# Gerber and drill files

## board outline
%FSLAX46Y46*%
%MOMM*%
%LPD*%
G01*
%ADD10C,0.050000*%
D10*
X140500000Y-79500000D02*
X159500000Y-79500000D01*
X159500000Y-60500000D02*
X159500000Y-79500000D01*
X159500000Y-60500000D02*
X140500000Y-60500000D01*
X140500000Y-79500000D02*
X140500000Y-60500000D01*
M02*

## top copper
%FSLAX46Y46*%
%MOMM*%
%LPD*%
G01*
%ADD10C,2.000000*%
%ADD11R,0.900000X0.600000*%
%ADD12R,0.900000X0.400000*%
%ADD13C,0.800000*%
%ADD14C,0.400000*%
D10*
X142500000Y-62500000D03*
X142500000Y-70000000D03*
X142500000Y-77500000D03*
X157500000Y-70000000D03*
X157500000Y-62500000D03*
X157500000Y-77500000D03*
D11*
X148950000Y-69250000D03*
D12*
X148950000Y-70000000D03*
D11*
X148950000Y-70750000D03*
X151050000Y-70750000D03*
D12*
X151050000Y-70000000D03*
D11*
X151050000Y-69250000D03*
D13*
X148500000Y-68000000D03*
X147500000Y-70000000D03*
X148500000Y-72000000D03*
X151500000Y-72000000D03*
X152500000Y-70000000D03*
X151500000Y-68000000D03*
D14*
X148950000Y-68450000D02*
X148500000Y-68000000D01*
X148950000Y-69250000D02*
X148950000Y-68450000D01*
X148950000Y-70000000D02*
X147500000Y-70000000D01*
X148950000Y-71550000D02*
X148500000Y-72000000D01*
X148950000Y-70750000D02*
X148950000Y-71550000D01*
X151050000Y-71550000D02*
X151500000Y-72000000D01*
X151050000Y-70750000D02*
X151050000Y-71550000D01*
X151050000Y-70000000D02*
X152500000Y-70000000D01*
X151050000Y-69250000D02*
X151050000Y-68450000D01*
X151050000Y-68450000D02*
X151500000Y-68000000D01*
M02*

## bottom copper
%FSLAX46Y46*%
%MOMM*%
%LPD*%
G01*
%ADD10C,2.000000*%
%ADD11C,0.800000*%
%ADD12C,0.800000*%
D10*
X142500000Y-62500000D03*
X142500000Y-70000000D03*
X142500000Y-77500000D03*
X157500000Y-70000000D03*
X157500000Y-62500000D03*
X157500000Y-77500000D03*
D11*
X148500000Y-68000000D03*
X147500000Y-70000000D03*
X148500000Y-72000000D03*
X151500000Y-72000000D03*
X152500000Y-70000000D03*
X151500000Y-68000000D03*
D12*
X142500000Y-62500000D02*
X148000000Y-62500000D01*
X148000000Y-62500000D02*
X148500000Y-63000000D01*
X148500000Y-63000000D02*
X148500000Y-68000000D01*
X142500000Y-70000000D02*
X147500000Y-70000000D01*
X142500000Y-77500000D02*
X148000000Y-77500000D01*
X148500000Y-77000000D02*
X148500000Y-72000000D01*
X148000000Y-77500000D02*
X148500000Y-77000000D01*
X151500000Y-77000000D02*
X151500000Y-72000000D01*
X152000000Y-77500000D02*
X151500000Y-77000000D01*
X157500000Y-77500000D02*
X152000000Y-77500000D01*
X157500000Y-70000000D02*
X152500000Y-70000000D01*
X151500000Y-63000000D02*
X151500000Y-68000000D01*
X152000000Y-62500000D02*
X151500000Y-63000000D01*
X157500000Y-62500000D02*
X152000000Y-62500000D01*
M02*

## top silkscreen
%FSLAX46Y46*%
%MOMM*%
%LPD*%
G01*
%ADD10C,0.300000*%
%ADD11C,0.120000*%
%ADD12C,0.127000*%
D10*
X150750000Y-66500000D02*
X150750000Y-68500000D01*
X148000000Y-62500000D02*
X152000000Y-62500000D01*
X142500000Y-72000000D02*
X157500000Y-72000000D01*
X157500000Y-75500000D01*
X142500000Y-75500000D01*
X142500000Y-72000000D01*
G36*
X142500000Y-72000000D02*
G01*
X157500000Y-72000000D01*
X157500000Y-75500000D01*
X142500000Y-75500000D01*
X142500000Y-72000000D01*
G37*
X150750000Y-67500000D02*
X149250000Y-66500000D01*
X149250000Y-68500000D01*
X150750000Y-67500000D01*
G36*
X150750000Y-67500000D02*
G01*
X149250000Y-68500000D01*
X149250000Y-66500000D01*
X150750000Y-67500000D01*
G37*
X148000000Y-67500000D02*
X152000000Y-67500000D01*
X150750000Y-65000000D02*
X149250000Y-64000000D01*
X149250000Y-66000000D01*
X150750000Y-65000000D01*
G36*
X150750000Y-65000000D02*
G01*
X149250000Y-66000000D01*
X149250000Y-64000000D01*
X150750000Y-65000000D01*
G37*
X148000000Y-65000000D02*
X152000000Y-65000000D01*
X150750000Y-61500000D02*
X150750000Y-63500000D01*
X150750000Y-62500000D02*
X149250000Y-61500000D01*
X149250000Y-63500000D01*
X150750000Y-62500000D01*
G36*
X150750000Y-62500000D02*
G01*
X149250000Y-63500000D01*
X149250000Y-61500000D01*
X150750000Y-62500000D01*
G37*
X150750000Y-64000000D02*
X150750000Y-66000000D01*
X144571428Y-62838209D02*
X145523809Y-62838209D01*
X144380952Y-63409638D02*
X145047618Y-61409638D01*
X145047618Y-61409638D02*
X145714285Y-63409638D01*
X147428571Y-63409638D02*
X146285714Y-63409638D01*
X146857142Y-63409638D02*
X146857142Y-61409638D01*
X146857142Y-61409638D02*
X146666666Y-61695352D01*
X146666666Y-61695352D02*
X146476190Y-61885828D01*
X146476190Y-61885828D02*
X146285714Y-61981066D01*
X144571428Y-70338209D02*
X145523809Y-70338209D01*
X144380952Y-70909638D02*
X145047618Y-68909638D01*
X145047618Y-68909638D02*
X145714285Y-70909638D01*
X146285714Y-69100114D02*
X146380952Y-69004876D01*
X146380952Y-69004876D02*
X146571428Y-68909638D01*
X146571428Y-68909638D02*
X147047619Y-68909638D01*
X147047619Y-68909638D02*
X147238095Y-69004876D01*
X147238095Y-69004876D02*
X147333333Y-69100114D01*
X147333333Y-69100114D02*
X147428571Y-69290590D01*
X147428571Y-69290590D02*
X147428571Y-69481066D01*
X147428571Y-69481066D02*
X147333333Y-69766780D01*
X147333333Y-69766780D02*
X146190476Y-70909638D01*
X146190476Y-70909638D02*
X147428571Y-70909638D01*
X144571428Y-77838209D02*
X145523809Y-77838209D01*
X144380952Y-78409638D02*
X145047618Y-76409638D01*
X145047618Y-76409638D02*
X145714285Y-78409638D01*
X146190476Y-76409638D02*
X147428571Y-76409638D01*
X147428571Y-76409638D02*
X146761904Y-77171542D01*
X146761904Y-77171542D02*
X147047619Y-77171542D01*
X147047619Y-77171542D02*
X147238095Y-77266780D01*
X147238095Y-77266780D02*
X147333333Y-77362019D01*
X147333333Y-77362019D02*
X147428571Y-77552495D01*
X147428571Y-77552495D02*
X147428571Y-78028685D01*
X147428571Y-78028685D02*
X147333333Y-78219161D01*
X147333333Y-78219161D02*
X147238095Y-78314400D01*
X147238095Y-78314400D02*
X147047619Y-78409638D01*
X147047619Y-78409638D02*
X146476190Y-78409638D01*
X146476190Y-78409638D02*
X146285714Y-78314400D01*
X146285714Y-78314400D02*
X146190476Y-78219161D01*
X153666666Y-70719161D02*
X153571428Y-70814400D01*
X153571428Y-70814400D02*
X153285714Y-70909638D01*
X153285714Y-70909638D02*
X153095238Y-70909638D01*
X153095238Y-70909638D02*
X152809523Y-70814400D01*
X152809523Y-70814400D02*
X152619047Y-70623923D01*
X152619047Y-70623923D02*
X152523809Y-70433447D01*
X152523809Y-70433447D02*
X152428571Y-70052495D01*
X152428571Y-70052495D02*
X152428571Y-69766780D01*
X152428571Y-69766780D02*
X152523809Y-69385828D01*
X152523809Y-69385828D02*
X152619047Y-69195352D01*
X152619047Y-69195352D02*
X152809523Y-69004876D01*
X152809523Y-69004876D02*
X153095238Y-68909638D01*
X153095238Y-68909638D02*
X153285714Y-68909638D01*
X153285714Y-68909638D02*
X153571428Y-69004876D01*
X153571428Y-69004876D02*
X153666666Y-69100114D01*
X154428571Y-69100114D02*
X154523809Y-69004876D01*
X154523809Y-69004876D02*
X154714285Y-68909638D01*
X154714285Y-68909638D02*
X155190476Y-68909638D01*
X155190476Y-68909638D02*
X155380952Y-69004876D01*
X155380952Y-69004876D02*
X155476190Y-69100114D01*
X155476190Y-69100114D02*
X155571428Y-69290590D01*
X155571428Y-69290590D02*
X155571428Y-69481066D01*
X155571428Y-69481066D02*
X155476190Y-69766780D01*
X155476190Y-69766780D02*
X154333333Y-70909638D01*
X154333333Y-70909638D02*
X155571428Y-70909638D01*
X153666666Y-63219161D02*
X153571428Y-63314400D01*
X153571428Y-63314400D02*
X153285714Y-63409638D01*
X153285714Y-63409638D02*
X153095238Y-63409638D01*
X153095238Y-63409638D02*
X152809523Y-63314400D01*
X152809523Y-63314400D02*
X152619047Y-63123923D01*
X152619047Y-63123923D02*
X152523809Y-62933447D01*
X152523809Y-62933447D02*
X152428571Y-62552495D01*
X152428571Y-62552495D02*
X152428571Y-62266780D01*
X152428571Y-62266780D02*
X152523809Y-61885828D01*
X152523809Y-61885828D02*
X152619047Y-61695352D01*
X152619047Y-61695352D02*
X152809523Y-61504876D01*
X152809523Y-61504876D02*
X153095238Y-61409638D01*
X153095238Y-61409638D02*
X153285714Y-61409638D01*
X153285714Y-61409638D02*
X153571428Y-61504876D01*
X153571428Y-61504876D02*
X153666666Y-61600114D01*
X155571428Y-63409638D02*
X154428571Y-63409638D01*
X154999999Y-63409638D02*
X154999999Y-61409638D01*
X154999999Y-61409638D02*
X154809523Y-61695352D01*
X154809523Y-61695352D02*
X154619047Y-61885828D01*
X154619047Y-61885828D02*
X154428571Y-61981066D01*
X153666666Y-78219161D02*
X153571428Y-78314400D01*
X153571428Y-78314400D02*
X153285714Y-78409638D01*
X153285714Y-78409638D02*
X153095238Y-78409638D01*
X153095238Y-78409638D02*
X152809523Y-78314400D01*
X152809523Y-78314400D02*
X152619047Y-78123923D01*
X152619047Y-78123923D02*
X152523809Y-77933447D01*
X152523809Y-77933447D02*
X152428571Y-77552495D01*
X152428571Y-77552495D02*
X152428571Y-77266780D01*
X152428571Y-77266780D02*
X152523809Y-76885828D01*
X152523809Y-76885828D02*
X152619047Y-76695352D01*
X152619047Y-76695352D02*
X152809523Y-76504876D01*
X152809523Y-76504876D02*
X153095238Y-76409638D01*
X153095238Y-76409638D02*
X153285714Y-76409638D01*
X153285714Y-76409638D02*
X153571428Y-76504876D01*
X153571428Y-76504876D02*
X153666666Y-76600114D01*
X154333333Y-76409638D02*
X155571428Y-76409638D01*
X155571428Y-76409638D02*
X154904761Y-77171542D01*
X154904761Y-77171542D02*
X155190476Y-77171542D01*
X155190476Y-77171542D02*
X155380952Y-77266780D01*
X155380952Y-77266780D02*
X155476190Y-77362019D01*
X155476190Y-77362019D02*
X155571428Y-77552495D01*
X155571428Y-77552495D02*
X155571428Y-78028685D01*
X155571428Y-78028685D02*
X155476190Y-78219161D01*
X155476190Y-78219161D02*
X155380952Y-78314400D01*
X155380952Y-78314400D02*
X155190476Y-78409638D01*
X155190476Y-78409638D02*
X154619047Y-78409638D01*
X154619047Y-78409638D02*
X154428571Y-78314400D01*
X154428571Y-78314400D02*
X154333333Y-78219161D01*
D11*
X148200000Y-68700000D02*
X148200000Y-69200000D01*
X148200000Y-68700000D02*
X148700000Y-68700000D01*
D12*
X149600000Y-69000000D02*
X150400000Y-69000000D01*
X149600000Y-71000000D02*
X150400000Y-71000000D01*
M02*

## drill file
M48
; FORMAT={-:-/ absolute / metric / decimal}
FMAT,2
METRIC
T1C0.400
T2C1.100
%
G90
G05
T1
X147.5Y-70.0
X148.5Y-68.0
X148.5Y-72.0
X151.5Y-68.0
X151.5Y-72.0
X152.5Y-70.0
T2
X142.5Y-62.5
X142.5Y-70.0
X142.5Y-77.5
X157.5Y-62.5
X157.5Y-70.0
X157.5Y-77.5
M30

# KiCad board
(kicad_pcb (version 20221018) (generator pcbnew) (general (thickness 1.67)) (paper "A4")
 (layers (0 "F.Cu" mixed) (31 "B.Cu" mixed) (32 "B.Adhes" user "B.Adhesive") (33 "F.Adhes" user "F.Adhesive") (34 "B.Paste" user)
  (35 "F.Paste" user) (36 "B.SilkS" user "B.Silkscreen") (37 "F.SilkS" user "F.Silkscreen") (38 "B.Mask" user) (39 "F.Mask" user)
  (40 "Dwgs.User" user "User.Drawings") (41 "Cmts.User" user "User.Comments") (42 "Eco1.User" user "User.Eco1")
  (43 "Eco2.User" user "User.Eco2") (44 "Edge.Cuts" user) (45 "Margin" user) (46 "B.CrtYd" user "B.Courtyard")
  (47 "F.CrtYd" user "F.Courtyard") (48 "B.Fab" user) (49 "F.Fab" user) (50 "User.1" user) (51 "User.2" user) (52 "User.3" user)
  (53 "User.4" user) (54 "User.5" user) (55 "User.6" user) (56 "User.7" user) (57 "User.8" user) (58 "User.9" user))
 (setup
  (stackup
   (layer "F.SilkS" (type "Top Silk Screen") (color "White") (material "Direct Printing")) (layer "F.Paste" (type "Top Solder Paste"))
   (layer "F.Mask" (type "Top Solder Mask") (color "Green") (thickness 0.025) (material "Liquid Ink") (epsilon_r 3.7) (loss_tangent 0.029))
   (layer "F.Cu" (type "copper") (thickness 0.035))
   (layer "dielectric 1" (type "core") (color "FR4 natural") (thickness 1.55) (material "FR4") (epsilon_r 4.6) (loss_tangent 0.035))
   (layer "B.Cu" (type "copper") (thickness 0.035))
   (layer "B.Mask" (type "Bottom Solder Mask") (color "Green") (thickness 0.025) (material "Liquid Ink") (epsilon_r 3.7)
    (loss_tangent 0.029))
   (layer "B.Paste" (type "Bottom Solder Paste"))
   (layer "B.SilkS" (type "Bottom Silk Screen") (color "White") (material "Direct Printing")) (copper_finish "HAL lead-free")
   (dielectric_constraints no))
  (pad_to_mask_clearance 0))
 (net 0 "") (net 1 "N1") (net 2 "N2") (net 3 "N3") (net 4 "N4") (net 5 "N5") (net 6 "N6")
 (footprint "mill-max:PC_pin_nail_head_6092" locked (layer "F.Cu") (at 142.5 62.5)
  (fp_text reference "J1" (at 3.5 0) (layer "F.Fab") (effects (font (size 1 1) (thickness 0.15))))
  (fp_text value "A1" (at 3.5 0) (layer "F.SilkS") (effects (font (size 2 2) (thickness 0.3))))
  (pad "1" thru_hole circle locked (at 0 0) (size 2 2) (drill 1.1) (layers "*.Cu" "*.Mask") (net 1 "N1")))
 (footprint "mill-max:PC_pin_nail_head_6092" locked (layer "F.Cu") (at 142.5 70)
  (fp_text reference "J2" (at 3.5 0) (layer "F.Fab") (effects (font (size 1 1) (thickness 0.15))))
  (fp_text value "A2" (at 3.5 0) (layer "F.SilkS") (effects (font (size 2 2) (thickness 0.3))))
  (pad "1" thru_hole circle locked (at 0 0) (size 2 2) (drill 1.1) (layers "*.Cu" "*.Mask") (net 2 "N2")))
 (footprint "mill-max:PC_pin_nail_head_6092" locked (layer "F.Cu") (at 142.5 77.5)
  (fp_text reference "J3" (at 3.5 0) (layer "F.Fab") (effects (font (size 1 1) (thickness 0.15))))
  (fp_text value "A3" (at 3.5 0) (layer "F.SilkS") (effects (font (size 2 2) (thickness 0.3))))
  (pad "1" thru_hole circle locked (at 0 0) (size 2 2) (drill 1.1) (layers "*.Cu" "*.Mask") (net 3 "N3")))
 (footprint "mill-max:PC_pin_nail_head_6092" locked (layer "F.Cu") (at 157.5 70)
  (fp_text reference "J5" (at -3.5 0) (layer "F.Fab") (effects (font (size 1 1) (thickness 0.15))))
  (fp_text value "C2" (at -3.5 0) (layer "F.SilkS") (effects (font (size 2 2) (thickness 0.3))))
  (pad "1" thru_hole circle locked (at 0 0) (size 2 2) (drill 1.1) (layers "*.Cu" "*.Mask") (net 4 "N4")))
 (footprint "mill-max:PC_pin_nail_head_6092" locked (layer "F.Cu") (at 157.5 62.5)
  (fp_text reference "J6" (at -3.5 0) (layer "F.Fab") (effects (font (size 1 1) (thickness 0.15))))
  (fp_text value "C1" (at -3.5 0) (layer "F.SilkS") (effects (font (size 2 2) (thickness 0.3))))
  (pad "1" thru_hole circle locked (at 0 0) (size 2 2) (drill 1.1) (layers "*.Cu" "*.Mask") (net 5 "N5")))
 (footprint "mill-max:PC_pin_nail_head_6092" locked (layer "F.Cu") (at 157.5 77.5)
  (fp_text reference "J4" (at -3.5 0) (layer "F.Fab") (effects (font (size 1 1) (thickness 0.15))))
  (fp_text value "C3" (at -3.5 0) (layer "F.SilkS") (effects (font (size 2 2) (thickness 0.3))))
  (pad "1" thru_hole circle locked (at 0 0) (size 2 2) (drill 1.1) (layers "*.Cu" "*.Mask") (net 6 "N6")))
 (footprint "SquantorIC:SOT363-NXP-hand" (layer "F.Cu") (at 150 70)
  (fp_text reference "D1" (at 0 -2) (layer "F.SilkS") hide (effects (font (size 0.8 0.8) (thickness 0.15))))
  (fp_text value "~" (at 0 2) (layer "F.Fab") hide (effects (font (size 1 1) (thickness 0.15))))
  (fp_line (start -1.8 -1.3) (end -1.8 -0.8) (stroke (width 0.12) (type solid)) (layer "F.SilkS"))
  (fp_line (start -1.8 -1.3) (end -1.3 -1.3) (stroke (width 0.12) (type solid)) (layer "F.SilkS"))
  (fp_line (start -0.4 -1) (end 0.4 -1) (stroke (width 0.127) (type solid)) (layer "F.SilkS"))
  (fp_line (start -0.4 1) (end 0.4 1) (stroke (width 0.127) (type solid)) (layer "F.SilkS"))
  (pad "1" smd rect (at -1.05 -0.75 270) (size 0.6 0.9) (layers "F.Cu" "F.Paste" "F.Mask") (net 1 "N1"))
  (pad "2" smd rect (at -1.05 0 270) (size 0.4 0.9) (layers "F.Cu" "F.Paste" "F.Mask") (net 2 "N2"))
  (pad "3" smd rect (at -1.05 0.75 270) (size 0.6 0.9) (layers "F.Cu" "F.Paste" "F.Mask") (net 3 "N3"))
  (pad "4" smd rect (at 1.05 0.75 270) (size 0.6 0.9) (layers "F.Cu" "F.Paste" "F.Mask") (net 6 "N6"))
  (pad "5" smd rect (at 1.05 0 270) (size 0.4 0.9) (layers "F.Cu" "F.Paste" "F.Mask") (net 4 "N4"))
  (pad "6" smd rect (at 1.05 -0.75 270) (size 0.6 0.9) (layers "F.Cu" "F.Paste" "F.Mask") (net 5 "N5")))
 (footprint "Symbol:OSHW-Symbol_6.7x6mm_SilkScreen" (layer "B.Cu") (at 150 69 180)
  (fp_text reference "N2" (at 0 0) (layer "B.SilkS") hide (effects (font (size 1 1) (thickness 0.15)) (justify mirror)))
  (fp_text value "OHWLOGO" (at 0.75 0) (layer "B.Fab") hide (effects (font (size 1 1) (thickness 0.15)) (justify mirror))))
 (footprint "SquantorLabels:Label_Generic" (layer "B.Cu") (at 150 72.5)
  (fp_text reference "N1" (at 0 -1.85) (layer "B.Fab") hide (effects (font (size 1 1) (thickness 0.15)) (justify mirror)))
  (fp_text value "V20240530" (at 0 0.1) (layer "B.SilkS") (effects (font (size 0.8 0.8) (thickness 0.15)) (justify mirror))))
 (gr_line (start 150.75 66.5) (end 150.75 68.5) (stroke (width 0.3) (type default)) (layer "F.SilkS"))
 (gr_line (start 148 62.5) (end 152 62.5) (stroke (width 0.3) (type default)) (layer "F.SilkS"))
 (gr_rect (start 142.5 72) (end 157.5 75.5) (stroke (width 0.3) (type solid)) (fill solid) (layer "F.SilkS"))
 (gr_poly (pts (xy 150.75 67.5) (xy 149.25 66.5) (xy 149.25 68.5)) (stroke (width 0.3) (type solid)) (fill solid) (layer "F.SilkS"))
 (gr_line (start 148 67.5) (end 152 67.5) (stroke (width 0.3) (type default)) (layer "F.SilkS"))
 (gr_poly (pts (xy 150.75 65) (xy 149.25 64) (xy 149.25 66)) (stroke (width 0.3) (type solid)) (fill solid) (layer "F.SilkS"))
 (gr_line (start 148 65) (end 152 65) (stroke (width 0.3) (type default)) (layer "F.SilkS"))
 (gr_line (start 150.75 61.5) (end 150.75 63.5) (stroke (width 0.3) (type default)) (layer "F.SilkS"))
 (gr_poly (pts (xy 150.75 62.5) (xy 149.25 61.5) (xy 149.25 63.5)) (stroke (width 0.3) (type solid)) (fill solid) (layer "F.SilkS"))
 (gr_line (start 150.75 64) (end 150.75 66) (stroke (width 0.3) (type default)) (layer "F.SilkS"))
 (gr_line (start 140.5 79.5) (end 159.5 79.5) (stroke (width 0.05) (type solid)) (layer "Edge.Cuts"))
 (gr_line (start 159.5 60.5) (end 159.5 79.5) (stroke (width 0.05) (type solid)) (layer "Edge.Cuts"))
 (gr_line (start 159.5 60.5) (end 140.5 60.5) (stroke (width 0.05) (type solid)) (layer "Edge.Cuts"))
 (gr_line (start 140.5 79.5) (end 140.5 60.5) (stroke (width 0.05) (type solid)) (layer "Edge.Cuts"))
 (segment (start 148.95 68.45) (end 148.5 68) (width 0.4) (layer "F.Cu") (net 1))
 (segment (start 148.95 69.25) (end 148.95 68.45) (width 0.4) (layer "F.Cu") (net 1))
 (via (at 148.5 68) (size 0.8) (drill 0.4) (layers "F.Cu" "B.Cu") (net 1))
 (segment (start 142.5 62.5) (end 148 62.5) (width 0.8) (layer "B.Cu") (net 1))
 (segment (start 148 62.5) (end 148.5 63) (width 0.8) (layer "B.Cu") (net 1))
 (segment (start 148.5 63) (end 148.5 68) (width 0.8) (layer "B.Cu") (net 1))
 (segment (start 148.95 70) (end 147.5 70) (width 0.4) (layer "F.Cu") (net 2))
 (via (at 147.5 70) (size 0.8) (drill 0.4) (layers "F.Cu" "B.Cu") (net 2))
 (segment (start 142.5 70) (end 147.5 70) (width 0.8) (layer "B.Cu") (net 2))
 (segment (start 148.95 71.55) (end 148.5 72) (width 0.4) (layer "F.Cu") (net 3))
 (segment (start 148.95 70.75) (end 148.95 71.55) (width 0.4) (layer "F.Cu") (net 3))
 (via (at 148.5 72) (size 0.8) (drill 0.4) (layers "F.Cu" "B.Cu") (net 3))
 (segment (start 142.5 77.5) (end 148 77.5) (width 0.8) (layer "B.Cu") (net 3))
 (segment (start 148.5 77) (end 148.5 72) (width 0.8) (layer "B.Cu") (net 3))
 (segment (start 148 77.5) (end 148.5 77) (width 0.8) (layer "B.Cu") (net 3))
 (segment (start 151.05 71.55) (end 151.5 72) (width 0.4) (layer "F.Cu") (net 6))
 (segment (start 151.05 70.75) (end 151.05 71.55) (width 0.4) (layer "F.Cu") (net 6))
 (via (at 151.5 72) (size 0.8) (drill 0.4) (layers "F.Cu" "B.Cu") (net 6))
 (segment (start 151.5 77) (end 151.5 72) (width 0.8) (layer "B.Cu") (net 6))
 (segment (start 152 77.5) (end 151.5 77) (width 0.8) (layer "B.Cu") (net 6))
 (segment (start 157.5 77.5) (end 152 77.5) (width 0.8) (layer "B.Cu") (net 6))
 (segment (start 151.05 70) (end 152.5 70) (width 0.4) (layer "F.Cu") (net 4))
 (via (at 152.5 70) (size 0.8) (drill 0.4) (layers "F.Cu" "B.Cu") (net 4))
 (segment (start 157.5 70) (end 152.5 70) (width 0.8) (layer "B.Cu") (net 4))
 (segment (start 151.05 69.25) (end 151.05 68.45) (width 0.4) (layer "F.Cu") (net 5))
 (segment (start 151.05 68.45) (end 151.5 68) (width 0.4) (layer "F.Cu") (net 5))
 (via (at 151.5 68) (size 0.8) (drill 0.4) (layers "F.Cu" "B.Cu") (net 5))
 (segment (start 151.5 63) (end 151.5 68) (width 0.8) (layer "B.Cu") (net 5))
 (segment (start 152 62.5) (end 151.5 63) (width 0.8) (layer "B.Cu") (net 5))
 (segment (start 157.5 62.5) (end 152 62.5) (width 0.8) (layer "B.Cu") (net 5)))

